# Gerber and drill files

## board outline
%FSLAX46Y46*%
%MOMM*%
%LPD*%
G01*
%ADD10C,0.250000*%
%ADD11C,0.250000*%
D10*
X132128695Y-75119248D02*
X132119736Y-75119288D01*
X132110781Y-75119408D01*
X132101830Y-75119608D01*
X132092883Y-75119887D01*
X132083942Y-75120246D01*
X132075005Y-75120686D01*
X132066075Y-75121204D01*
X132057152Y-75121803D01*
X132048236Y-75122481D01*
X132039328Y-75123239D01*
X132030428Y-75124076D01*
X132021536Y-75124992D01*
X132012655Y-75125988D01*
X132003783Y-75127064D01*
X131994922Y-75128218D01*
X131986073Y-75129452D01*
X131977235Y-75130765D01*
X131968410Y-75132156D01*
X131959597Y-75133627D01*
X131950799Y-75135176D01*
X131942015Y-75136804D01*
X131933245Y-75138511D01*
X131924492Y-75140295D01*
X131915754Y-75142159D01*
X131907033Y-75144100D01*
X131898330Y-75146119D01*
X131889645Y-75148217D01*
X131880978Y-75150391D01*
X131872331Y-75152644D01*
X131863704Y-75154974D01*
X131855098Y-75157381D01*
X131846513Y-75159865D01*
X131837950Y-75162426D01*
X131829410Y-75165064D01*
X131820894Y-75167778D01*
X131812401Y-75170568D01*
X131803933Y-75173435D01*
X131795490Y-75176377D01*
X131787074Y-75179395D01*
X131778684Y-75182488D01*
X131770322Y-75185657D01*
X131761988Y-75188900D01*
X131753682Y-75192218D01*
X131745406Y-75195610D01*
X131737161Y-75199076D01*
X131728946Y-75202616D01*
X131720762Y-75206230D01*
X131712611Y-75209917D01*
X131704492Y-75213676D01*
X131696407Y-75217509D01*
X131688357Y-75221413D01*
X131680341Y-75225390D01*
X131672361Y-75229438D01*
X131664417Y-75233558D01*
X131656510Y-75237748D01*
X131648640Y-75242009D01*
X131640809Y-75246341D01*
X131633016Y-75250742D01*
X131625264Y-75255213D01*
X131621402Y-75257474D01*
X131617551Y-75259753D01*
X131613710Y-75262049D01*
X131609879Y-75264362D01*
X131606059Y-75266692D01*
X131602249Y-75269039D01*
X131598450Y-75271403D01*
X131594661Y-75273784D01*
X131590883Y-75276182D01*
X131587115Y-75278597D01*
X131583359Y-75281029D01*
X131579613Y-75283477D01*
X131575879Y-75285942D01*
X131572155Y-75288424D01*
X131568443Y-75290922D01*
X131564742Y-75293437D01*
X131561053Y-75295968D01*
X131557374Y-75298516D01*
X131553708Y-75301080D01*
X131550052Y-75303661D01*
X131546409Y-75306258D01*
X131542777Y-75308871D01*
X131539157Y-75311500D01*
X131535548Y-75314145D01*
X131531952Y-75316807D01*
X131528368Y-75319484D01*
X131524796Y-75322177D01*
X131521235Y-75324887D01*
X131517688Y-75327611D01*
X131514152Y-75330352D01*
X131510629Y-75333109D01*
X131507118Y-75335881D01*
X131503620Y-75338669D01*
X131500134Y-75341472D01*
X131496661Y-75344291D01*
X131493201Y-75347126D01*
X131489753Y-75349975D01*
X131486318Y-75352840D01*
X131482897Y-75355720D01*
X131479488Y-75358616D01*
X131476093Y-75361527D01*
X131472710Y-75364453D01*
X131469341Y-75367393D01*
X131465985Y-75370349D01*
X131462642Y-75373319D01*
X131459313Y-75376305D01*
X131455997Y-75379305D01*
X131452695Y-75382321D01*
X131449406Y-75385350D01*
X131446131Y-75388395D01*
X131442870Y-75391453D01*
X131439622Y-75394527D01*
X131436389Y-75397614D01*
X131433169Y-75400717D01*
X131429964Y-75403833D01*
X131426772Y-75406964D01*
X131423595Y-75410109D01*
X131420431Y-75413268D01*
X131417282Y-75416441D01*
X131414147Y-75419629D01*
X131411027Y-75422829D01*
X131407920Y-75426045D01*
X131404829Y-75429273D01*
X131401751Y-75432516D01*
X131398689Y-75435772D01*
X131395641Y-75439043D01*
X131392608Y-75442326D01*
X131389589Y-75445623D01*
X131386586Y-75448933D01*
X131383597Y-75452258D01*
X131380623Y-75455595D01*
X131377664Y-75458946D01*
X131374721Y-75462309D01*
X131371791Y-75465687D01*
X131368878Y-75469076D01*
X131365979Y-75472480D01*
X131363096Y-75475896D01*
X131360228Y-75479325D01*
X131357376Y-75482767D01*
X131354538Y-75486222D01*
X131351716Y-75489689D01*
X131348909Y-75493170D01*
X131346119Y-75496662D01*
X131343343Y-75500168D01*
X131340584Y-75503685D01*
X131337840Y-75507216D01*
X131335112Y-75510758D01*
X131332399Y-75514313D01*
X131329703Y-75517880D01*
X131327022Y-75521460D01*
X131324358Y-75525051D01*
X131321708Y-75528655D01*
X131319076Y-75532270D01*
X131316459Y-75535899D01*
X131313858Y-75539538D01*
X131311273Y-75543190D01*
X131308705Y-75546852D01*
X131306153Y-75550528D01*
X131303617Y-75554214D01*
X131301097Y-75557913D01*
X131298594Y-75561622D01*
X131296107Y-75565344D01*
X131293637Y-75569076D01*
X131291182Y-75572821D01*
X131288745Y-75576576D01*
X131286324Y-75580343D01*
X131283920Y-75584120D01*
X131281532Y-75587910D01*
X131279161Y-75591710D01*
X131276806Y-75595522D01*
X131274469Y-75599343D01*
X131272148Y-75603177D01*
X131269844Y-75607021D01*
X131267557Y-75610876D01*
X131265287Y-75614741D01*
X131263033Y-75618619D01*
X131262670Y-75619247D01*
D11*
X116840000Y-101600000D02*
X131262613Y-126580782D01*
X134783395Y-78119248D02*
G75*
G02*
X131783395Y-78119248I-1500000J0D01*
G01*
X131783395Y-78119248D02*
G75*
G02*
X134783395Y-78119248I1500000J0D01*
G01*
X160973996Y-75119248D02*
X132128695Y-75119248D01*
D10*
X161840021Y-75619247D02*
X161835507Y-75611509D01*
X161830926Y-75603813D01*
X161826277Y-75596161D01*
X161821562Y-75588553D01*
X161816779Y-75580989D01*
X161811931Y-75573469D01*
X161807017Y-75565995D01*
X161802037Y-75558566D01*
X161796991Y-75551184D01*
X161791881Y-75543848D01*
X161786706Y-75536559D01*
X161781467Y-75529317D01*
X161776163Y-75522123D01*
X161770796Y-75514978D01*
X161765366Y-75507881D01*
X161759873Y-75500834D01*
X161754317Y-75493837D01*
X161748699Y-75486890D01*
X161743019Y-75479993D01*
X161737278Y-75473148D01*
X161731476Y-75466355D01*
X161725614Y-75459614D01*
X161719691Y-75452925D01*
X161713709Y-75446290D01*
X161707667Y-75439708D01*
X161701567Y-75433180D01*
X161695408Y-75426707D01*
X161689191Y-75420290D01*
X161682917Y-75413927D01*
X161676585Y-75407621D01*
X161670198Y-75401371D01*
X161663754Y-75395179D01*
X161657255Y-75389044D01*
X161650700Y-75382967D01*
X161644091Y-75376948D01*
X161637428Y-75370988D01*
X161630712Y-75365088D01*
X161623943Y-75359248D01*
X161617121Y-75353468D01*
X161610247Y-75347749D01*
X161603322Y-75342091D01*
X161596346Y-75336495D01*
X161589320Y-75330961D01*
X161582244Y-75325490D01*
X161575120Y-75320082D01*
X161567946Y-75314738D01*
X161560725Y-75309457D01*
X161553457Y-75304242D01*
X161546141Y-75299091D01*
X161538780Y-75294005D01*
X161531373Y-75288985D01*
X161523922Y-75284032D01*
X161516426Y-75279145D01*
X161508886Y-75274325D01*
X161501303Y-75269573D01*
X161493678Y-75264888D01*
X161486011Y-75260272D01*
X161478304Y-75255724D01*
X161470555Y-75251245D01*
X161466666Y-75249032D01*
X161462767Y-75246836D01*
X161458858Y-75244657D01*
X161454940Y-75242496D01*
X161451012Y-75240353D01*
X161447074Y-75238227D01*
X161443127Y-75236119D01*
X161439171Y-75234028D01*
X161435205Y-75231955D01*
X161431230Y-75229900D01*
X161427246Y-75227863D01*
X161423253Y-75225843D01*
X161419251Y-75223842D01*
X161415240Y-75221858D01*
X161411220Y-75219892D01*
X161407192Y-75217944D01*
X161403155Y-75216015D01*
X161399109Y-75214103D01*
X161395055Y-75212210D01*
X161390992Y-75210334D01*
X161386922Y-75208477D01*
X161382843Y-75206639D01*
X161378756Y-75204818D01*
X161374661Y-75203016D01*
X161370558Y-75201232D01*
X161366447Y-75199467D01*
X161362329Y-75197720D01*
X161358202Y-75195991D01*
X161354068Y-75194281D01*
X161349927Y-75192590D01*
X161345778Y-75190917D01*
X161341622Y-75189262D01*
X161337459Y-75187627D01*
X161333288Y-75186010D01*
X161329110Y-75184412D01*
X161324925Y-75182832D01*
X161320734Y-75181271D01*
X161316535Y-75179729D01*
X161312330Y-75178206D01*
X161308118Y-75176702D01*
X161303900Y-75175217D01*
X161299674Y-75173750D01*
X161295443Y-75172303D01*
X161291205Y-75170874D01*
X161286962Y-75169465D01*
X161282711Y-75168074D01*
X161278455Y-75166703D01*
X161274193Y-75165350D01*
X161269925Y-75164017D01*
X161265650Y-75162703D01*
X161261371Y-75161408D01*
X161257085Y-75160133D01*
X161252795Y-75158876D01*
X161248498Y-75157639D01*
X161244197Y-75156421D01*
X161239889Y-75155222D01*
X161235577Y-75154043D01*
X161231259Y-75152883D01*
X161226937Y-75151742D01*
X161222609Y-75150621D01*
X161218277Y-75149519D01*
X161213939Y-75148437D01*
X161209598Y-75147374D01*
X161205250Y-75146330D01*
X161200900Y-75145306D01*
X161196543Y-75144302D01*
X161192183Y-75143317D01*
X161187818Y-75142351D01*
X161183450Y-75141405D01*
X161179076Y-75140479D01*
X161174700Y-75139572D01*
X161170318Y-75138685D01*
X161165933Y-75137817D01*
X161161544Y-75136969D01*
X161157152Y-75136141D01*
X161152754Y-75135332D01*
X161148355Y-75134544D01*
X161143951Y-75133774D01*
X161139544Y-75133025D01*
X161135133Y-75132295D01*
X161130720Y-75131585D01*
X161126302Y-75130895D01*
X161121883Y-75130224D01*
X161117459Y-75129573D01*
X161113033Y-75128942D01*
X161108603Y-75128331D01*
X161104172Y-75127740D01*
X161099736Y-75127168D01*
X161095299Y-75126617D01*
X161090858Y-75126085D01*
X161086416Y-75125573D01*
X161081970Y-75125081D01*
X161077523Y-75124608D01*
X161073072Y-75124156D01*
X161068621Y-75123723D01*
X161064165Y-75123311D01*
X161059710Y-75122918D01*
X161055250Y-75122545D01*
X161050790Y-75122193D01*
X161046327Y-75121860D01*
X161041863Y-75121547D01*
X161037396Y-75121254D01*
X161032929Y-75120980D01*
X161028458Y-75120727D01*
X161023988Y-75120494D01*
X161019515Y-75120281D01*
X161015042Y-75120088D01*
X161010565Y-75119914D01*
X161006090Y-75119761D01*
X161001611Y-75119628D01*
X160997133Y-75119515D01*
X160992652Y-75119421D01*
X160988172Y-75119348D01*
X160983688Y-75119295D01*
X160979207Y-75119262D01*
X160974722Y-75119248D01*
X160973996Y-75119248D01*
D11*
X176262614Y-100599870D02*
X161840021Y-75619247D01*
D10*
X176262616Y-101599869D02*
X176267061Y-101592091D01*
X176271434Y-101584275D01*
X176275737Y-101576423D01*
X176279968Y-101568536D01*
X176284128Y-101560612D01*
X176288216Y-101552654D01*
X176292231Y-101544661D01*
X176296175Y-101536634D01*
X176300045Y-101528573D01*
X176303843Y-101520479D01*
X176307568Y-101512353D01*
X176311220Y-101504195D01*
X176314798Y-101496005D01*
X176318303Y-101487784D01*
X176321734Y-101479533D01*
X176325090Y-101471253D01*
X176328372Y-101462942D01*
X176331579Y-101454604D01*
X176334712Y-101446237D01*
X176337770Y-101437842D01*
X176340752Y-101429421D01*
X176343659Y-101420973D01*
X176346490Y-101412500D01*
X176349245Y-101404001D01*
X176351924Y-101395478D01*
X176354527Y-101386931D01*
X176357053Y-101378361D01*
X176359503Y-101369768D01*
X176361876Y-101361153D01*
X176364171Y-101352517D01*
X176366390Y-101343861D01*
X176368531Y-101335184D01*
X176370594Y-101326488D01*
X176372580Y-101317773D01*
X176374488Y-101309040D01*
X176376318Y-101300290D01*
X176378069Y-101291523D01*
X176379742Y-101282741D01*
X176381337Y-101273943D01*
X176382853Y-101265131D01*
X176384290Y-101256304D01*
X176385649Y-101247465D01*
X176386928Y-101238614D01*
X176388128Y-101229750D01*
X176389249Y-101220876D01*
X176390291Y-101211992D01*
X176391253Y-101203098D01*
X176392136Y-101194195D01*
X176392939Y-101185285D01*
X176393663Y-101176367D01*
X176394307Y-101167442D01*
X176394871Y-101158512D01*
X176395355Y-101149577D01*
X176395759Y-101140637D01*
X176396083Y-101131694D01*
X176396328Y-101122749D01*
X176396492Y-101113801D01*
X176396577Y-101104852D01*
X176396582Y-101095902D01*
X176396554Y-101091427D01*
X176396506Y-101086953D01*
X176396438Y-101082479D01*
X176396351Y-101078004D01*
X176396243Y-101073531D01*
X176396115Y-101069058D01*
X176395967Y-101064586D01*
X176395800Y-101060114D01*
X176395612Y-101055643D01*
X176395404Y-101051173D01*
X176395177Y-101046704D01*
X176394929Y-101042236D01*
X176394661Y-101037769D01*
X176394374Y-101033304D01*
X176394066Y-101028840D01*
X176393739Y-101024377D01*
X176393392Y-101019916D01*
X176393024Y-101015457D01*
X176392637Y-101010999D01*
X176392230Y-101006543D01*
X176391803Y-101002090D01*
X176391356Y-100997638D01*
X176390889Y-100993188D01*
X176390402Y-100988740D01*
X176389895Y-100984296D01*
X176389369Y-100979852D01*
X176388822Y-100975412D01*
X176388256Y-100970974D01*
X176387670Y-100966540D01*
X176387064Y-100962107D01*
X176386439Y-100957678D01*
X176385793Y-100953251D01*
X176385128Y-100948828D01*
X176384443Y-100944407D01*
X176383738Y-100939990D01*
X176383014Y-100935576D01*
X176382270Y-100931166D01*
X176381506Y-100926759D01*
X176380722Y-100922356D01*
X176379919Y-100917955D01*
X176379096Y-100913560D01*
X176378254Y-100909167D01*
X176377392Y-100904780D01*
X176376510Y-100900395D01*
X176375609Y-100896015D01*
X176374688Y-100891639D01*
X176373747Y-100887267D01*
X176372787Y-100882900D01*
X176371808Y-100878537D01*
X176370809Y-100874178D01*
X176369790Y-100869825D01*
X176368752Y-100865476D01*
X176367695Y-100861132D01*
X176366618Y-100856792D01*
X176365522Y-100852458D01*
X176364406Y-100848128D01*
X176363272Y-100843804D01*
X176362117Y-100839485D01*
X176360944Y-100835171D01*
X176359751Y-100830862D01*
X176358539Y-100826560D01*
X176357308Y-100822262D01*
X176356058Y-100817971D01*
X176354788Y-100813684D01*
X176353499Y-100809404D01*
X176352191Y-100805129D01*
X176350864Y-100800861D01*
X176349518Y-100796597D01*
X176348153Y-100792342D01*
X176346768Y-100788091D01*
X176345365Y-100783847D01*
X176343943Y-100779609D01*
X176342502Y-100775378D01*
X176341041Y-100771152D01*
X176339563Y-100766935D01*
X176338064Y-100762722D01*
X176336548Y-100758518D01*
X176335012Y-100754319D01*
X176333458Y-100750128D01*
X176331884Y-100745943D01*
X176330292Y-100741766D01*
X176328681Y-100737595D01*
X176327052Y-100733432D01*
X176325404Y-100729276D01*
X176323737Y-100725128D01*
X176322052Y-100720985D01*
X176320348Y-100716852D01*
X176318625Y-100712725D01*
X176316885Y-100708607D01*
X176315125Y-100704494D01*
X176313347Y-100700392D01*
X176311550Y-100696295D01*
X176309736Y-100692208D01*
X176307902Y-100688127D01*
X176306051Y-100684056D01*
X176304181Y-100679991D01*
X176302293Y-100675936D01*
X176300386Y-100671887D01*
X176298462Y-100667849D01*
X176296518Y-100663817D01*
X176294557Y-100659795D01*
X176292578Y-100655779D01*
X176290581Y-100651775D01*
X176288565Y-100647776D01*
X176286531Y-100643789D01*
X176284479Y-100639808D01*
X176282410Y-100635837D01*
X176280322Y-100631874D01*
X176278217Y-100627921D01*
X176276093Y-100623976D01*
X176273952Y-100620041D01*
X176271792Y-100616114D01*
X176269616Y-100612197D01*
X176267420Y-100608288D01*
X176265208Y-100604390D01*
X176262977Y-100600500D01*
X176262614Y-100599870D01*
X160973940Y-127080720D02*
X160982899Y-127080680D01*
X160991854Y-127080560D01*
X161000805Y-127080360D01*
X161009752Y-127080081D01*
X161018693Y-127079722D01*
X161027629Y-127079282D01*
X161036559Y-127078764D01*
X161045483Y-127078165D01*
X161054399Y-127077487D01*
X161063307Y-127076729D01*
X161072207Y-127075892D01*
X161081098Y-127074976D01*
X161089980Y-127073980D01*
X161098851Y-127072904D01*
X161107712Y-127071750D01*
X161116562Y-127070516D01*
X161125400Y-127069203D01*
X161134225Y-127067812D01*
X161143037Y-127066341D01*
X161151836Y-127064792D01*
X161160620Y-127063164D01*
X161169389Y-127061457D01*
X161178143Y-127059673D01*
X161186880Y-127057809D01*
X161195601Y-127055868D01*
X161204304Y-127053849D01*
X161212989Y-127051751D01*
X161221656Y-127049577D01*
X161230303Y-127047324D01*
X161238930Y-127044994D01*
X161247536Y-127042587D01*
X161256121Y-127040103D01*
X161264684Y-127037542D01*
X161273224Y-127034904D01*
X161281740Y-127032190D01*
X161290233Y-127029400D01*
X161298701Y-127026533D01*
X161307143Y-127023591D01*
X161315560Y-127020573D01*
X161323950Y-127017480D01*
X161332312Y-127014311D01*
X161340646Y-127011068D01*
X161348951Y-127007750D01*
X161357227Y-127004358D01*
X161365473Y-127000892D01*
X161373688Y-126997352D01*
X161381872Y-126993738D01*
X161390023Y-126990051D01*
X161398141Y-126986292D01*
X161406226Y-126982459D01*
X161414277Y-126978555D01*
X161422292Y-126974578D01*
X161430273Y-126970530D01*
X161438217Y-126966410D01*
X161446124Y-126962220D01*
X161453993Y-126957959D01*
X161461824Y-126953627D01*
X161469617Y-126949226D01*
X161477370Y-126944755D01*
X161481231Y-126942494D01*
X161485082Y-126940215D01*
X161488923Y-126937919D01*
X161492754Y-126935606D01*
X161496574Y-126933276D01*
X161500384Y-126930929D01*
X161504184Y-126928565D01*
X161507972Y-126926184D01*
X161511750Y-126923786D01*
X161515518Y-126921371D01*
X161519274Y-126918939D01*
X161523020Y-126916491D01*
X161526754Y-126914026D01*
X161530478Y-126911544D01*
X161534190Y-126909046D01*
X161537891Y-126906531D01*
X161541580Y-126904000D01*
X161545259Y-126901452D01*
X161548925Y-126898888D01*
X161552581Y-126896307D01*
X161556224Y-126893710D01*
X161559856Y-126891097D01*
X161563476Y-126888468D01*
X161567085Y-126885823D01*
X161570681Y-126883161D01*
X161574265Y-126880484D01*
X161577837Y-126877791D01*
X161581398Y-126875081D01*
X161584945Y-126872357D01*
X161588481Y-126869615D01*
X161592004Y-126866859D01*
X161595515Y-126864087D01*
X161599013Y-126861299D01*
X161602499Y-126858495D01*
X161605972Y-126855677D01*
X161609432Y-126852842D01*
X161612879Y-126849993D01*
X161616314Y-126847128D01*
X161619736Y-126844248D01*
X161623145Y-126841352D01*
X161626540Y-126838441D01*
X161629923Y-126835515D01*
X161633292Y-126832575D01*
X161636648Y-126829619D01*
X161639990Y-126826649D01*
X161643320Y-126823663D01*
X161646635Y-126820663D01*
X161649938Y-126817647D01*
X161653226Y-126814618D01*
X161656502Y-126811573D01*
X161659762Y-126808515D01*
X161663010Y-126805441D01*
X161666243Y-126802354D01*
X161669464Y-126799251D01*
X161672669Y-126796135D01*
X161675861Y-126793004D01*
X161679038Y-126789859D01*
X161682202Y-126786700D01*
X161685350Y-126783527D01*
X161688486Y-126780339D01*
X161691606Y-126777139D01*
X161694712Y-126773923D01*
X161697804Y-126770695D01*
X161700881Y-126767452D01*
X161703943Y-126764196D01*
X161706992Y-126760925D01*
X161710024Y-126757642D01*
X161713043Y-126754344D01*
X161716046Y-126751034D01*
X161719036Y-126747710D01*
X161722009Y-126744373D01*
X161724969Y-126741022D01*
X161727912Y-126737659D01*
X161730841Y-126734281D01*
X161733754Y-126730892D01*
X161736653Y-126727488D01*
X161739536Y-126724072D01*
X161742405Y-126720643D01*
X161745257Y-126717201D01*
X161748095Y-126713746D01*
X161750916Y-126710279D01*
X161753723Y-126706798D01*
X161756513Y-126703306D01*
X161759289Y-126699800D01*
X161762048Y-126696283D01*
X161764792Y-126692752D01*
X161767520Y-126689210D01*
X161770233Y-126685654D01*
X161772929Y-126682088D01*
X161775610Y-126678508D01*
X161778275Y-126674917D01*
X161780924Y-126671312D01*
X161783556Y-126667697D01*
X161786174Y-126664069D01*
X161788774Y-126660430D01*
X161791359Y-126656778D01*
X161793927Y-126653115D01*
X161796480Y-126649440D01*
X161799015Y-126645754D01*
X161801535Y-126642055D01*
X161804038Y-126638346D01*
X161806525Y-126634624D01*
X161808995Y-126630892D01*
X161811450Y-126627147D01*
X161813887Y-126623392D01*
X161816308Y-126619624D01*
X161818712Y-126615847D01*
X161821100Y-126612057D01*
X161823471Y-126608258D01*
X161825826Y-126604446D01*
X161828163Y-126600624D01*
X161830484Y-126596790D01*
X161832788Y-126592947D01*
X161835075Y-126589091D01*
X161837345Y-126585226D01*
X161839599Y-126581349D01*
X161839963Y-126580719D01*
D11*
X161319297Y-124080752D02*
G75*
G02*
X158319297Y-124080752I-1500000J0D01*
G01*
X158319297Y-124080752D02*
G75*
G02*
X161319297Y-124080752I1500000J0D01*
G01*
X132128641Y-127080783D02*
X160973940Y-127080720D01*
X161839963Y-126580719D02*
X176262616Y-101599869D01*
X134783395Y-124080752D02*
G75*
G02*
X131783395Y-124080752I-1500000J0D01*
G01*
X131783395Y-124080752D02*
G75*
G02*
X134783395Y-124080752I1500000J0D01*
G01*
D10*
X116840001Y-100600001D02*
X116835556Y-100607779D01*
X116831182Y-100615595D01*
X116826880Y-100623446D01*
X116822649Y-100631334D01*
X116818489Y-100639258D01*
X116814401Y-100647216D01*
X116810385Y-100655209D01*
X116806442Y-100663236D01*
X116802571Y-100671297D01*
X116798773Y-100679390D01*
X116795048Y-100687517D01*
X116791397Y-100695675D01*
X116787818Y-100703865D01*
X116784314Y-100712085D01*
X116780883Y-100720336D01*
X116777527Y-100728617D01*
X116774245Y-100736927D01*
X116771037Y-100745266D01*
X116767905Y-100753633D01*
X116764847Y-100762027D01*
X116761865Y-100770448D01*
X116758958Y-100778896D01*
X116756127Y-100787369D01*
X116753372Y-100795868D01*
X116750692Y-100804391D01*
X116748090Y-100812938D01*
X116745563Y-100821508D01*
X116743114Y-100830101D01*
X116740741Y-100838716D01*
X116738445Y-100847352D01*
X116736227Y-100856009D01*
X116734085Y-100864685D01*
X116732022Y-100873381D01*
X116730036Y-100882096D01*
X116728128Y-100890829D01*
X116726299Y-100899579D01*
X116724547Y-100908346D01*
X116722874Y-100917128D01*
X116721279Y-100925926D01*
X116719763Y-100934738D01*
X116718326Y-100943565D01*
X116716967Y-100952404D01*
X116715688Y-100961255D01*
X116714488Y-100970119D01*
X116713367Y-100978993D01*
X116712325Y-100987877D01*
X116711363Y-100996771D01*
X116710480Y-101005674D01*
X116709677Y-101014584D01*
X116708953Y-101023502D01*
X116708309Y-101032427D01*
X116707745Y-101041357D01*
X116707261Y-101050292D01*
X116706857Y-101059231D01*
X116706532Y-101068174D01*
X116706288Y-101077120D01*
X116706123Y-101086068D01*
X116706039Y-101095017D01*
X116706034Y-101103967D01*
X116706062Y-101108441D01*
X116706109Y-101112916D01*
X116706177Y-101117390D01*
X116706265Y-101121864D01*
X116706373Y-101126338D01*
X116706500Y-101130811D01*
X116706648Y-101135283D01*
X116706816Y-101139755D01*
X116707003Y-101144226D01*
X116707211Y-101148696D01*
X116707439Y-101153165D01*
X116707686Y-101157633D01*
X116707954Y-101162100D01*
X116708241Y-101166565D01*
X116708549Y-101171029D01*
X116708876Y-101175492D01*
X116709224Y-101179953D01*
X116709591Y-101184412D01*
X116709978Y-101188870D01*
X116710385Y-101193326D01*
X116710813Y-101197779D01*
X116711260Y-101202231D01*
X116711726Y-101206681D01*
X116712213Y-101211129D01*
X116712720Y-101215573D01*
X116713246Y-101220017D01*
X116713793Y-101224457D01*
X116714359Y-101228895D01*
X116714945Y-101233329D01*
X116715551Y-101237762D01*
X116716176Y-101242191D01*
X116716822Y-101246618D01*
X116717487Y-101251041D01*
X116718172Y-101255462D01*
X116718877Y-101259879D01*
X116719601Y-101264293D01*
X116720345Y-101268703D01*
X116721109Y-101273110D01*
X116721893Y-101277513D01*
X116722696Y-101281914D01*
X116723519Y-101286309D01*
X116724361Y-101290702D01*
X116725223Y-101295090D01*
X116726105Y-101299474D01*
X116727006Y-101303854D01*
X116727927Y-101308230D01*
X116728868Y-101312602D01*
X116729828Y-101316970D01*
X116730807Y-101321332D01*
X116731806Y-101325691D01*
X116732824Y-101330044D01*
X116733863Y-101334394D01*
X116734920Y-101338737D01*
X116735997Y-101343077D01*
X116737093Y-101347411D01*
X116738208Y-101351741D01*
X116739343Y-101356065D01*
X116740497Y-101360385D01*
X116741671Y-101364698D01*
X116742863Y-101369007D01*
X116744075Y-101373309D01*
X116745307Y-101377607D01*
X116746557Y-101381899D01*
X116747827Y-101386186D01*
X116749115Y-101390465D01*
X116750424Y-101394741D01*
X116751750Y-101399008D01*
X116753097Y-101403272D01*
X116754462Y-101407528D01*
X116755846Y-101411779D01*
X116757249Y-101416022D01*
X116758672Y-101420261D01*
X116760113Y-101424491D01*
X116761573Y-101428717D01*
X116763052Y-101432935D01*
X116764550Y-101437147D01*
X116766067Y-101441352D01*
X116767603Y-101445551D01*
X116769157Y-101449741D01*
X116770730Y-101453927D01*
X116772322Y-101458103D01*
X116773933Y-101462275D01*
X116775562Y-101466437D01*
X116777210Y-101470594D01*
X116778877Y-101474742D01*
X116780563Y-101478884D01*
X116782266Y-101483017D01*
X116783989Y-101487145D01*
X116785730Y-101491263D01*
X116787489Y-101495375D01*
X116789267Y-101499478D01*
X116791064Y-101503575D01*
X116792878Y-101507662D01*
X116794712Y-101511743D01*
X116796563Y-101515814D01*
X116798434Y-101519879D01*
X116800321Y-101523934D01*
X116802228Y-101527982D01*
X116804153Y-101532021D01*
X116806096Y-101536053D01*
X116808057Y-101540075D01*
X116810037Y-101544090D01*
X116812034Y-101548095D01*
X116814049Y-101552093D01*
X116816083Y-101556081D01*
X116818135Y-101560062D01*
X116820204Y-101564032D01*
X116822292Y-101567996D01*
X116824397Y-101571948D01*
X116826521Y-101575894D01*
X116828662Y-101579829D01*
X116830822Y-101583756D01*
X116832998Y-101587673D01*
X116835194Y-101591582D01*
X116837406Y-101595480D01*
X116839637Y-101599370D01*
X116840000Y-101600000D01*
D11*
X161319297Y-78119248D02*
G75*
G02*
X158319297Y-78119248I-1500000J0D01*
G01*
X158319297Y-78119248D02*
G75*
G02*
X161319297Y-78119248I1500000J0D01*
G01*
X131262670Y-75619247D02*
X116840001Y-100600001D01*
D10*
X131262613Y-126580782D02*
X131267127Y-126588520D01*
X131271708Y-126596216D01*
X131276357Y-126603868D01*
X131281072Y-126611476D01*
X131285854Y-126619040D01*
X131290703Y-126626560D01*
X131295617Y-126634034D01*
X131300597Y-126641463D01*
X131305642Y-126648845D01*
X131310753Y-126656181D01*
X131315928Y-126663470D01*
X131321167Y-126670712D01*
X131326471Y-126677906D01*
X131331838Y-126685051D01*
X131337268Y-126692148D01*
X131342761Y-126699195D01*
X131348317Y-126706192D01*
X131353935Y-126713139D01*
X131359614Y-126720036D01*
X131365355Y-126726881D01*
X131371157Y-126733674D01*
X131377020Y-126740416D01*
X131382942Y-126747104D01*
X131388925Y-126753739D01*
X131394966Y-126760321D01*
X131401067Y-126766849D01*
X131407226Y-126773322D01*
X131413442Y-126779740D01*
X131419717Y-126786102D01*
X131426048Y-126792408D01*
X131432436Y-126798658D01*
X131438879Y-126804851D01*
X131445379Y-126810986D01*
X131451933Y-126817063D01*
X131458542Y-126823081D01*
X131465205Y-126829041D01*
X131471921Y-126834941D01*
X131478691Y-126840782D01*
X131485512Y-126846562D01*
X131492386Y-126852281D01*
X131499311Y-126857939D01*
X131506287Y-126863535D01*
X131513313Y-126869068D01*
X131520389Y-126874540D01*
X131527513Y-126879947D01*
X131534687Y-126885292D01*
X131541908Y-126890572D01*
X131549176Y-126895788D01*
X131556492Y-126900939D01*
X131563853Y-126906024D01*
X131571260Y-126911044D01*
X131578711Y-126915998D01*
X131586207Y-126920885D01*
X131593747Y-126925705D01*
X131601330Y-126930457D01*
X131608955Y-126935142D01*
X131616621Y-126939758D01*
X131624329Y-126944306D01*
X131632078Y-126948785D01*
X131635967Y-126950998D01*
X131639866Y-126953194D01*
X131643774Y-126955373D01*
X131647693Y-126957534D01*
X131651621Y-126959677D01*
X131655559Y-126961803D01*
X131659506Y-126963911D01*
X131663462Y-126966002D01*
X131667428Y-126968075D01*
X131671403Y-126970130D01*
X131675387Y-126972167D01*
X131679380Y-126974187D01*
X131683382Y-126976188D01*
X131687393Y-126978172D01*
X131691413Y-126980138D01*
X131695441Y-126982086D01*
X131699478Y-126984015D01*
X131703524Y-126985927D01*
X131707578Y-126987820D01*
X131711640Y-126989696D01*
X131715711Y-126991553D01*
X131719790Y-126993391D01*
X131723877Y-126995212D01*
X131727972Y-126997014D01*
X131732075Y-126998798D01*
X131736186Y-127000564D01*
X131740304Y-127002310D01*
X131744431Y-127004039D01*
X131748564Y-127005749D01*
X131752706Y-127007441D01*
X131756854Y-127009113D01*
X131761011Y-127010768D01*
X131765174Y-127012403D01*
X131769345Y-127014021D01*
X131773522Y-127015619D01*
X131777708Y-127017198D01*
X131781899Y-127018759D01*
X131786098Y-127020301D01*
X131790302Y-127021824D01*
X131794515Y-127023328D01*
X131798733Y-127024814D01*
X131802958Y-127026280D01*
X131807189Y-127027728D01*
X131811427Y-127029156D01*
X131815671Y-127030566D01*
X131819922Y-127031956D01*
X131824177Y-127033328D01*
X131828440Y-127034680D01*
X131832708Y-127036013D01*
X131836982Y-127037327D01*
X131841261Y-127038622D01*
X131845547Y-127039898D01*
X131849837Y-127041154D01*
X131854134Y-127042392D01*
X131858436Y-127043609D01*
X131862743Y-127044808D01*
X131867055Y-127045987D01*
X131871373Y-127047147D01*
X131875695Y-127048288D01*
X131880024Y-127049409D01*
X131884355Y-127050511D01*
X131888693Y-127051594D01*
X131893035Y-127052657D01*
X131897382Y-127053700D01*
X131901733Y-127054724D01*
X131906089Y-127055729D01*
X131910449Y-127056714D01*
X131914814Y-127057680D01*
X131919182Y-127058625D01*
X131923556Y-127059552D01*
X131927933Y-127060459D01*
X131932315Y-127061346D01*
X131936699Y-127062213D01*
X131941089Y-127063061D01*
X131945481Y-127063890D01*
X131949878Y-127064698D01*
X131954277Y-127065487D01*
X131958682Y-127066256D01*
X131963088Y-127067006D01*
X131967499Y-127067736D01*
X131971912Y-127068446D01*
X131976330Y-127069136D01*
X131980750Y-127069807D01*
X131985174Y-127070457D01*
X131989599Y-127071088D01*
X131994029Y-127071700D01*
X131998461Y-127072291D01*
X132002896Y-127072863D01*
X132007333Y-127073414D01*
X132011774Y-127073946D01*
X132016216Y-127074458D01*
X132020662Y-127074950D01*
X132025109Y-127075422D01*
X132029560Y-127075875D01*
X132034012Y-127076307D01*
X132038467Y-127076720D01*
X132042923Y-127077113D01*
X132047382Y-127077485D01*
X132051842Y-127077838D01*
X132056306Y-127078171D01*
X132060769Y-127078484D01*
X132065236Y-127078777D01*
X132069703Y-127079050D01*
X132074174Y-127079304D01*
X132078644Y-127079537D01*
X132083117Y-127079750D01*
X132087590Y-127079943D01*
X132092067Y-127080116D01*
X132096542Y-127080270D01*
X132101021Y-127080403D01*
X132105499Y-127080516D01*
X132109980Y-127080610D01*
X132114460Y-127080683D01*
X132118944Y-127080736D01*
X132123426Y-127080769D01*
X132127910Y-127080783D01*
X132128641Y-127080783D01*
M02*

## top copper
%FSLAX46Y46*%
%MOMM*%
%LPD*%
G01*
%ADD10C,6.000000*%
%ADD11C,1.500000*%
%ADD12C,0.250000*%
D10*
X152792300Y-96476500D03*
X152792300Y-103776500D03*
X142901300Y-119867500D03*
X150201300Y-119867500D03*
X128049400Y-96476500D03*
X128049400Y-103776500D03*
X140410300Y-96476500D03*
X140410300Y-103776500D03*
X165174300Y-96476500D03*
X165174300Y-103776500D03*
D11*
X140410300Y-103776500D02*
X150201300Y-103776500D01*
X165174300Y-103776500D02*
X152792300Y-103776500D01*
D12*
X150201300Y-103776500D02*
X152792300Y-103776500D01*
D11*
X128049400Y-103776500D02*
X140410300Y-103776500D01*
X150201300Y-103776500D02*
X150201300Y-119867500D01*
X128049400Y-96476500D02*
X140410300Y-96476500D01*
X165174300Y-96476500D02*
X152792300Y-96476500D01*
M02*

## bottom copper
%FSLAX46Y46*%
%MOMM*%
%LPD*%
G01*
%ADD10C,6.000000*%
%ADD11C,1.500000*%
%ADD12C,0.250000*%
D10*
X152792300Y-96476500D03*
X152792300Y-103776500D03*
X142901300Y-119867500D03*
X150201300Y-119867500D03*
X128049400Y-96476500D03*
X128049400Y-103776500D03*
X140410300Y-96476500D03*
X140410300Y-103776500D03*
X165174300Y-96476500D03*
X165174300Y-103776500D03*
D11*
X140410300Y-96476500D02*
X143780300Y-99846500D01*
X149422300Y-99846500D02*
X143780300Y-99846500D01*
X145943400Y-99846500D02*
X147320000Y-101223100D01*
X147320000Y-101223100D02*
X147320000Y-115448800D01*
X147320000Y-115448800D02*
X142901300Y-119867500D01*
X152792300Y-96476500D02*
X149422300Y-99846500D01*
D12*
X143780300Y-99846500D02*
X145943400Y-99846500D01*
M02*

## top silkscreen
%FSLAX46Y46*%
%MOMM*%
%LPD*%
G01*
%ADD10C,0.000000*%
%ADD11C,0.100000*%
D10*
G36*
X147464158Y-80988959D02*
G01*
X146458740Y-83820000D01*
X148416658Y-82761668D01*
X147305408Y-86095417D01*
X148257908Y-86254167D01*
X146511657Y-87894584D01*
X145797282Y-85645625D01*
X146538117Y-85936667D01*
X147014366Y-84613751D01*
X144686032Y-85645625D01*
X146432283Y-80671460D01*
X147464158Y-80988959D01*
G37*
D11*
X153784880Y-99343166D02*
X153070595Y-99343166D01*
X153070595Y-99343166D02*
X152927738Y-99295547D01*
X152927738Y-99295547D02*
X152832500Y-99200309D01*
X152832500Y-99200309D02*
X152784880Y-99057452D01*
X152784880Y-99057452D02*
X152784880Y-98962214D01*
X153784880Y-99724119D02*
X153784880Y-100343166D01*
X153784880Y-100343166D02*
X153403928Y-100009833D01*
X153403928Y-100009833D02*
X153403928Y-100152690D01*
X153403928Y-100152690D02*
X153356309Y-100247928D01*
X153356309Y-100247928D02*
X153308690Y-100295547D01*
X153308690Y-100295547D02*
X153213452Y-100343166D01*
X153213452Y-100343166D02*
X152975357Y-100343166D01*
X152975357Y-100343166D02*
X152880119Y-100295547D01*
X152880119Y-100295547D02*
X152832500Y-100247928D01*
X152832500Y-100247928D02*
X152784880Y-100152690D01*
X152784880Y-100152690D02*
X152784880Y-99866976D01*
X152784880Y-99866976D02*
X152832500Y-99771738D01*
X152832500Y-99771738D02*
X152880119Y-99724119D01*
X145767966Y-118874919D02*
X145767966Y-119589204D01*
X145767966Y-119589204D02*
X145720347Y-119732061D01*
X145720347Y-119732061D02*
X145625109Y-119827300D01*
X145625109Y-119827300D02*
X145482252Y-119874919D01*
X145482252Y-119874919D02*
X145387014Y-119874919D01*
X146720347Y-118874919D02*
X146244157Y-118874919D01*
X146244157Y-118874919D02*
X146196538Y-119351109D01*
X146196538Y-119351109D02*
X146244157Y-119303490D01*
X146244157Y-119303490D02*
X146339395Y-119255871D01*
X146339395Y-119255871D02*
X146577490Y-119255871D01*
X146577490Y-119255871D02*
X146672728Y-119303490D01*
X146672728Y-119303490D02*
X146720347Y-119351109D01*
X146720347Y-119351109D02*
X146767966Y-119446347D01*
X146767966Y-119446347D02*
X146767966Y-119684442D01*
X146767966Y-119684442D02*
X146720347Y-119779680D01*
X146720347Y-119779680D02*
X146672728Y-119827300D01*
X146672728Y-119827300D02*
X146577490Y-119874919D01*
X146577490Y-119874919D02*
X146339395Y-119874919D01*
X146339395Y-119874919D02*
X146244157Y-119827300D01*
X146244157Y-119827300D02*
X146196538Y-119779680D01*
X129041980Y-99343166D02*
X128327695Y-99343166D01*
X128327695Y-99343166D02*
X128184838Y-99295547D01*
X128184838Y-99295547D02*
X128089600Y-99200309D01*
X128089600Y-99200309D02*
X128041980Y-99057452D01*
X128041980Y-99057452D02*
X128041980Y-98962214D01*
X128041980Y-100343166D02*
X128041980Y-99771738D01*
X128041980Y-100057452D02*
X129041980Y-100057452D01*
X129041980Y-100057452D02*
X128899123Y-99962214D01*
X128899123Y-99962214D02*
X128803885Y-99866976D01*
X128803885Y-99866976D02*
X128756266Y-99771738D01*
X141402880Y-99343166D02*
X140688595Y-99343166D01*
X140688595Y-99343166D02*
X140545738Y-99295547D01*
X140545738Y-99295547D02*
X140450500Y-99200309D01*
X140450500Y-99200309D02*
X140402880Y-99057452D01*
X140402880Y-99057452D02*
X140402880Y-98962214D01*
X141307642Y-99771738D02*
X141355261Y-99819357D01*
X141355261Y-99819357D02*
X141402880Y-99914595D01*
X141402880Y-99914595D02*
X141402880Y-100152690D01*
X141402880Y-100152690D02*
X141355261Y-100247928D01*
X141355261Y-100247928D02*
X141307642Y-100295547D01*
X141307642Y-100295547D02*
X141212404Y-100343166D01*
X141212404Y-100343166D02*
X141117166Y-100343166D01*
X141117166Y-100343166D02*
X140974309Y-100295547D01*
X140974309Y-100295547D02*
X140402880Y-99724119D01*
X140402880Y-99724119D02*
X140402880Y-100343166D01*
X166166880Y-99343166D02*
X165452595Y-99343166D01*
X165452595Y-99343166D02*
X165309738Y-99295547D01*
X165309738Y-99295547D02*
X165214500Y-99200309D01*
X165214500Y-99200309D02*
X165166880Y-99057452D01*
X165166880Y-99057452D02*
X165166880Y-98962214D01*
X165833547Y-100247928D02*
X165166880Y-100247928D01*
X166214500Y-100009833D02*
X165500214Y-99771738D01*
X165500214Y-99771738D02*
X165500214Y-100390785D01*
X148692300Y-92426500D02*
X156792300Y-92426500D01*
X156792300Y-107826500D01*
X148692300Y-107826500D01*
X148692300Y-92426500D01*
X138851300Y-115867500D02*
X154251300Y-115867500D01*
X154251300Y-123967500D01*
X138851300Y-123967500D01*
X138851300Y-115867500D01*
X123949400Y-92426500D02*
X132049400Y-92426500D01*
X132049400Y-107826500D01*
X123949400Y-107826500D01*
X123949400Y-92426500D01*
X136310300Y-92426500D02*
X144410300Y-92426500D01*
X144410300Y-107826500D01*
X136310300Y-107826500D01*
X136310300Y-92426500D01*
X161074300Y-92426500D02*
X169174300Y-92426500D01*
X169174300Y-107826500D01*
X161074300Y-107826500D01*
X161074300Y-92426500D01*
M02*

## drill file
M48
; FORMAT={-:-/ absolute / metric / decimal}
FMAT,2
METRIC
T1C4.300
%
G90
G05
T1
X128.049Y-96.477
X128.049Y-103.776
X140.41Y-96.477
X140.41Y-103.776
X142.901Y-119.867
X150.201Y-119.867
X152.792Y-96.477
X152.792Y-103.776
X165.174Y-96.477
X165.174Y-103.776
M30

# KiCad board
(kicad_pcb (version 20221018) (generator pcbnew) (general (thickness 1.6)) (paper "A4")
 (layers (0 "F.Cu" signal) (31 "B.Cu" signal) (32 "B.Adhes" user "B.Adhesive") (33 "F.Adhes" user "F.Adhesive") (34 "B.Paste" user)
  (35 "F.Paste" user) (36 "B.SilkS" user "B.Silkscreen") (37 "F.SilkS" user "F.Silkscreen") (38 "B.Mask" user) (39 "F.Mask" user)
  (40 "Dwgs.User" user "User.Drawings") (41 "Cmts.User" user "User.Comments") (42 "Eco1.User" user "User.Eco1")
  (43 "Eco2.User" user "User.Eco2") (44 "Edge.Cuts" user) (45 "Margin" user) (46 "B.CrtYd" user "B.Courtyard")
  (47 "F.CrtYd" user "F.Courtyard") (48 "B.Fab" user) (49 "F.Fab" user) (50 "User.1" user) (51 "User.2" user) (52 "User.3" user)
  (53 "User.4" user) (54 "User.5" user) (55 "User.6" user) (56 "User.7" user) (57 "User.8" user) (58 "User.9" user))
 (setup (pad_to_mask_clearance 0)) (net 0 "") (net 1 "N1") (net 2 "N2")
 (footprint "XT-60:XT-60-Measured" (layer "F.Cu") (at 152.7423 100.1265 -90)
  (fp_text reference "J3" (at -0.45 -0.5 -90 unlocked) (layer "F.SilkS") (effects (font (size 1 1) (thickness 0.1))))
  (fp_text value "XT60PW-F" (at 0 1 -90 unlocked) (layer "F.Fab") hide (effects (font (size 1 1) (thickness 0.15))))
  (fp_rect (start -7.7 -4.05) (end 7.7 4.05) (stroke (width 0.1) (type default)) (fill none) (layer "F.SilkS"))
  (pad "1" thru_hole circle (at -3.65 -0.05 270) (size 6 6) (drill 4.3) (layers "*.Cu" "*.Mask") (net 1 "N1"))
  (pad "2" thru_hole circle (at 3.65 -0.05 270) (size 6 6) (drill 4.3) (layers "*.Cu" "*.Mask") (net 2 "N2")))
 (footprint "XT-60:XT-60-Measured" (layer "F.Cu") (at 146.5513 119.9175)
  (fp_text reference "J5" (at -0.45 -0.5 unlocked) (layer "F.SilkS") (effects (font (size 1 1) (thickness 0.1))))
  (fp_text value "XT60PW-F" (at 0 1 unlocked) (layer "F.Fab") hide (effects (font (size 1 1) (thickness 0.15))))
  (fp_rect (start -7.7 -4.05) (end 7.7 4.05) (stroke (width 0.1) (type default)) (fill none) (layer "F.SilkS"))
  (pad "1" thru_hole circle (at -3.65 -0.05) (size 6 6) (drill 4.3) (layers "*.Cu" "*.Mask") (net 1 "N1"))
  (pad "2" thru_hole circle (at 3.65 -0.05) (size 6 6) (drill 4.3) (layers "*.Cu" "*.Mask") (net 2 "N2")))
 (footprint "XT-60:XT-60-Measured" (layer "F.Cu") (at 127.9994 100.1265 -90)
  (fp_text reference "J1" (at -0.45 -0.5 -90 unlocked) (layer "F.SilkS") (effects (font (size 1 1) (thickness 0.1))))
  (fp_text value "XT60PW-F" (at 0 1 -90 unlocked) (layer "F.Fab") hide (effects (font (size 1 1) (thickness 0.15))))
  (fp_rect (start -7.7 -4.05) (end 7.7 4.05) (stroke (width 0.1) (type default)) (fill none) (layer "F.SilkS"))
  (pad "1" thru_hole circle (at -3.65 -0.05 270) (size 6 6) (drill 4.3) (layers "*.Cu" "*.Mask") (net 1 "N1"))
  (pad "2" thru_hole circle (at 3.65 -0.05 270) (size 6 6) (drill 4.3) (layers "*.Cu" "*.Mask") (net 2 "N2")))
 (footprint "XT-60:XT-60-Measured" (layer "F.Cu") (at 140.3603 100.1265 -90)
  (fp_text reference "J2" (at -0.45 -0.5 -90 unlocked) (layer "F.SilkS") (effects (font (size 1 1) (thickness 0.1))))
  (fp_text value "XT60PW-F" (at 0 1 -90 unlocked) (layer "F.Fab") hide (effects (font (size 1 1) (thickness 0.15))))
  (fp_rect (start -7.7 -4.05) (end 7.7 4.05) (stroke (width 0.1) (type default)) (fill none) (layer "F.SilkS"))
  (pad "1" thru_hole circle (at -3.65 -0.05 270) (size 6 6) (drill 4.3) (layers "*.Cu" "*.Mask") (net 1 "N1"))
  (pad "2" thru_hole circle (at 3.65 -0.05 270) (size 6 6) (drill 4.3) (layers "*.Cu" "*.Mask") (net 2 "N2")))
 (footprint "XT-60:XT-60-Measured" (layer "F.Cu") (at 165.1243 100.1265 -90)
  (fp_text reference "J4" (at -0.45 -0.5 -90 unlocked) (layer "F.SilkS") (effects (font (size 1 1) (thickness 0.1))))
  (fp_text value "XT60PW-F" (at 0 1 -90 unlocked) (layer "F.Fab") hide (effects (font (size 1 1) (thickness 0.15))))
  (fp_rect (start -7.7 -4.05) (end 7.7 4.05) (stroke (width 0.1) (type default)) (fill none) (layer "F.SilkS"))
  (pad "1" thru_hole circle (at -3.65 -0.05 270) (size 6 6) (drill 4.3) (layers "*.Cu" "*.Mask") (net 1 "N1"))
  (pad "2" thru_hole circle (at 3.65 -0.05 270) (size 6 6) (drill 4.3) (layers "*.Cu" "*.Mask") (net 2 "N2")))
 (gr_poly
  (pts (xy 147.464158 80.988959) (xy 146.45874 83.82) (xy 148.416658 82.761668) (xy 147.305408 86.095417) (xy 148.257908 86.254167)
   (xy 146.511657 87.894584) (xy 145.797282 85.645625) (xy 146.538117 85.936667) (xy 147.014366 84.613751) (xy 144.686032 85.645625)
   (xy 146.432283 80.67146))
  (stroke (width 0) (type solid)) (fill solid) (layer "F.SilkS"))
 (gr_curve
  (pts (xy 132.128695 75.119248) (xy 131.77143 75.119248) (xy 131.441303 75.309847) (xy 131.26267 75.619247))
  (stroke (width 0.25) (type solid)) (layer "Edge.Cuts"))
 (gr_line (start 116.84 101.6) (end 131.262613 126.580782) (stroke (width 0.25) (type solid)) (layer "Edge.Cuts"))
 (gr_circle (center 133.283395 78.119248) (end 134.783395 78.119248) (stroke (width 0.25) (type solid)) (fill none) (layer "Edge.Cuts"))
 (gr_line (start 160.973996 75.119248) (end 132.128695 75.119248) (stroke (width 0.25) (type solid)) (layer "Edge.Cuts"))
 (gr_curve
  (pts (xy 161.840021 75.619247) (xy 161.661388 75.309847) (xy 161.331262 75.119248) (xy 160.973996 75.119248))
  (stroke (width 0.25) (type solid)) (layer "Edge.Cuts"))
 (gr_line (start 176.262614 100.59987) (end 161.840021 75.619247) (stroke (width 0.25) (type solid)) (layer "Edge.Cuts"))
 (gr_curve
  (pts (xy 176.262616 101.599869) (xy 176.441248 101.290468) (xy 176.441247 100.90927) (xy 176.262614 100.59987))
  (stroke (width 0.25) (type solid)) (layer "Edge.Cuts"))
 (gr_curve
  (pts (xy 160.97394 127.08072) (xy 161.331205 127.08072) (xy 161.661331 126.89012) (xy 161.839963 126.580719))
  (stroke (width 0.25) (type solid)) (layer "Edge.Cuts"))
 (gr_circle (center 159.819297 124.080752) (end 161.319297 124.080752) (stroke (width 0.25) (type solid)) (fill none) (layer "Edge.Cuts"))
 (gr_line (start 132.128641 127.080783) (end 160.97394 127.08072) (stroke (width 0.25) (type solid)) (layer "Edge.Cuts"))
 (gr_line (start 161.839963 126.580719) (end 176.262616 101.599869) (stroke (width 0.25) (type solid)) (layer "Edge.Cuts"))
 (gr_circle (center 133.283395 124.080752) (end 134.783395 124.080752) (stroke (width 0.25) (type solid)) (fill none) (layer "Edge.Cuts"))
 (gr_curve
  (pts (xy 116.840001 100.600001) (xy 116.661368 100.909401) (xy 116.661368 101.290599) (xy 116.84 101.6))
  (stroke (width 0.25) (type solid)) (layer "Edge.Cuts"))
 (gr_circle (center 159.819297 78.119248) (end 161.319297 78.119248) (stroke (width 0.25) (type solid)) (fill none) (layer "Edge.Cuts"))
 (gr_line (start 131.26267 75.619247) (end 116.840001 100.600001) (stroke (width 0.25) (type solid)) (layer "Edge.Cuts"))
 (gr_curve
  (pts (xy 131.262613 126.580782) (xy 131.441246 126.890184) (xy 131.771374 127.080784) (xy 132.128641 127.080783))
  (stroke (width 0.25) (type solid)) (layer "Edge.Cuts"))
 (segment (start 140.4103 103.7765) (end 150.2013 103.7765) (width 1.5) (layer "F.Cu") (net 2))
 (segment (start 165.1743 103.7765) (end 152.7923 103.7765) (width 1.5) (layer "F.Cu") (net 2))
 (segment (start 150.2013 103.7765) (end 152.7923 103.7765) (width 0.25) (layer "F.Cu") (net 2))
 (segment (start 128.0494 103.7765) (end 140.4103 103.7765) (width 1.5) (layer "F.Cu") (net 2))
 (segment (start 150.2013 103.7765) (end 150.2013 119.8675) (width 1.5) (layer "F.Cu") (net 2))
 (segment (start 128.0494 96.4765) (end 140.4103 96.4765) (width 1.5) (layer "F.Cu") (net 1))
 (segment (start 165.1743 96.4765) (end 152.7923 96.4765) (width 1.5) (layer "F.Cu") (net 1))
 (segment (start 140.4103 96.4765) (end 143.7803 99.8465) (width 1.5) (layer "B.Cu") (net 1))
 (segment (start 149.4223 99.8465) (end 143.7803 99.8465) (width 1.5) (layer "B.Cu") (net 1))
 (segment (start 145.9434 99.8465) (end 147.32 101.2231) (width 1.5) (layer "B.Cu") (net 1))
 (segment (start 147.32 101.2231) (end 147.32 115.4488) (width 1.5) (layer "B.Cu") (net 1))
 (segment (start 147.32 115.4488) (end 142.9013 119.8675) (width 1.5) (layer "B.Cu") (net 1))
 (segment (start 152.7923 96.4765) (end 149.4223 99.8465) (width 1.5) (layer "B.Cu") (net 1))
 (segment (start 143.7803 99.8465) (end 145.9434 99.8465) (width 0.25) (layer "B.Cu") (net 1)))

